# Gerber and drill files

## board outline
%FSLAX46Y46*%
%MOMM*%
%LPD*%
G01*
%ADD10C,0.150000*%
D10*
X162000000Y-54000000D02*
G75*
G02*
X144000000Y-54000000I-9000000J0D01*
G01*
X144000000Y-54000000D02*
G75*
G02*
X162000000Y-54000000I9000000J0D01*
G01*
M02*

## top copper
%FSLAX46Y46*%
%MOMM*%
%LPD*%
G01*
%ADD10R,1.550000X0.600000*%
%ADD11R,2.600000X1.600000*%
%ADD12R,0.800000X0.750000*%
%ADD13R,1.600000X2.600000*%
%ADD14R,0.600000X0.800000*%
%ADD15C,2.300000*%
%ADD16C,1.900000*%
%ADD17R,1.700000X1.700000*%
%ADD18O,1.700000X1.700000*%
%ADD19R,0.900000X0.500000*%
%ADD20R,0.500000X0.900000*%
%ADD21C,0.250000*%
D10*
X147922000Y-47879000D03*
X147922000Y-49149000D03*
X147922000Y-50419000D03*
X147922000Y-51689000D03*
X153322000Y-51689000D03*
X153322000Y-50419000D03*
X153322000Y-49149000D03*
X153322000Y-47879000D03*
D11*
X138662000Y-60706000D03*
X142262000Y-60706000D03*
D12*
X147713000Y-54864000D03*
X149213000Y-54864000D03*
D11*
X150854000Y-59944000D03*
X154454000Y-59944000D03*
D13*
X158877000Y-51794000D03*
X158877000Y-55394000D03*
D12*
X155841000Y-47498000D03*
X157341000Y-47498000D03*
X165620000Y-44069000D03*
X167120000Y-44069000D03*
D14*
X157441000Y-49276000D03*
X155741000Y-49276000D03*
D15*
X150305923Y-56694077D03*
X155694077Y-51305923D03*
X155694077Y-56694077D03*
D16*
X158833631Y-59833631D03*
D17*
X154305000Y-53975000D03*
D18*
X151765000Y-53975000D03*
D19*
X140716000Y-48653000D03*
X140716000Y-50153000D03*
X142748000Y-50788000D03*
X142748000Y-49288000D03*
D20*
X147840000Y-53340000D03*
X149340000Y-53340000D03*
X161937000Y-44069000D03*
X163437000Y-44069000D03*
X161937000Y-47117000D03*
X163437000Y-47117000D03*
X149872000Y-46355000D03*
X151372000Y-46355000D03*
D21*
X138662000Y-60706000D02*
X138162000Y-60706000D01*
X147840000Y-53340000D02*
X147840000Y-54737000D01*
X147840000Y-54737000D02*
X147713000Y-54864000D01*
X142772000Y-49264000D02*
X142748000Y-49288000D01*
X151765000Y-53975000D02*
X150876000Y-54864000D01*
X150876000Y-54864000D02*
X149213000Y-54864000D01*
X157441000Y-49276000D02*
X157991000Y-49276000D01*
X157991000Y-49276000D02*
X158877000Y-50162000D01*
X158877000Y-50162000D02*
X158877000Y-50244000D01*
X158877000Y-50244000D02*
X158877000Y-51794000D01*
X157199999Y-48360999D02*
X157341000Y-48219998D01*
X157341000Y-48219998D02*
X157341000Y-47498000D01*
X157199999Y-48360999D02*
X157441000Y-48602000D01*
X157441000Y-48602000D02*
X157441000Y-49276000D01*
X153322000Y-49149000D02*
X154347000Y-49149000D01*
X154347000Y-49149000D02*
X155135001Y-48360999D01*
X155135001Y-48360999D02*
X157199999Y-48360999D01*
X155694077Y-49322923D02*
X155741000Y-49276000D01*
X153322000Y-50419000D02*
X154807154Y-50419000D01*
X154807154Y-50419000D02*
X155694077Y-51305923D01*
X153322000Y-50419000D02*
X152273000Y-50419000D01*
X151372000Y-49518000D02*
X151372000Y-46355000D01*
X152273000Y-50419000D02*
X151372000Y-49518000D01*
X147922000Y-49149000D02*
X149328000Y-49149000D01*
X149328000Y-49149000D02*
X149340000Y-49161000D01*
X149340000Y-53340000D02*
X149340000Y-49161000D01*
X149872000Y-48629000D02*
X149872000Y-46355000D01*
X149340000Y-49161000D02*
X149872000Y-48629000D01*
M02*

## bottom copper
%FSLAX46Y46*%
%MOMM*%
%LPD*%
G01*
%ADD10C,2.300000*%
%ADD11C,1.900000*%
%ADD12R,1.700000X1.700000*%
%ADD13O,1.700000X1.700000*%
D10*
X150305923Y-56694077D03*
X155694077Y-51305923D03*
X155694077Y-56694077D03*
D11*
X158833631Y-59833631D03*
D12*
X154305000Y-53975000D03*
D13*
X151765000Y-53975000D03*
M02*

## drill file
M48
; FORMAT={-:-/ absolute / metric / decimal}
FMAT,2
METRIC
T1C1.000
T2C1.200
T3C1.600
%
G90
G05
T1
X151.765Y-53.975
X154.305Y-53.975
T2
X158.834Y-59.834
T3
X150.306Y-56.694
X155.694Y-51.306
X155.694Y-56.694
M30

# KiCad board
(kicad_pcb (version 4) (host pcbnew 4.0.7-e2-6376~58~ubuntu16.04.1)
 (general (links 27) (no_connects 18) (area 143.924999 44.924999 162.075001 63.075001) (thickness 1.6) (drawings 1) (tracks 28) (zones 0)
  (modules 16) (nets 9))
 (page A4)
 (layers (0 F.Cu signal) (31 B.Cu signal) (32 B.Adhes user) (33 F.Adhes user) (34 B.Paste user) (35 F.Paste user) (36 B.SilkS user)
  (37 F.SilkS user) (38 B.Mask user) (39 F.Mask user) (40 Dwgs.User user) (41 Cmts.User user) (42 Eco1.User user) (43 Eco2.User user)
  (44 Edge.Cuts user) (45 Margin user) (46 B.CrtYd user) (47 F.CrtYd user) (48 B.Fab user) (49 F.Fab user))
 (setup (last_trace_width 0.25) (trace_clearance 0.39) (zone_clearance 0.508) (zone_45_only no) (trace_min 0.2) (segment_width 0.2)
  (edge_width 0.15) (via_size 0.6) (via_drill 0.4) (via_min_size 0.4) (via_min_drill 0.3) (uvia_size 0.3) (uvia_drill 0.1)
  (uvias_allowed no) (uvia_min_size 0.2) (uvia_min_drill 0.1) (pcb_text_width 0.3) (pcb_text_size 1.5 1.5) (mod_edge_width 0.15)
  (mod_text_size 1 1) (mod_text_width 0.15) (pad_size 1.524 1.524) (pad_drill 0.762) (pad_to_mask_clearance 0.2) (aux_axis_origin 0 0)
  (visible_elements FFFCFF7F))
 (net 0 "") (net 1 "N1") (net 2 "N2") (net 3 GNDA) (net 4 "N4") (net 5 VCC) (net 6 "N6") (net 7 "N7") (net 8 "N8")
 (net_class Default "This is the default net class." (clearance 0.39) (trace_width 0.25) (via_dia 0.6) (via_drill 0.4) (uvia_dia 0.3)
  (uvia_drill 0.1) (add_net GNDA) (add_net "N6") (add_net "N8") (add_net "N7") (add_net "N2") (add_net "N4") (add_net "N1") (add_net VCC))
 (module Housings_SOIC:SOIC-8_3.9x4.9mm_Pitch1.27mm (layer F.Cu) (at 150.622 49.784)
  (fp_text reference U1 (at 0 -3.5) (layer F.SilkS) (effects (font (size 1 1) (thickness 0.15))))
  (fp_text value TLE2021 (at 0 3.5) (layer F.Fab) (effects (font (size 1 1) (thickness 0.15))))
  (pad 1 smd rect (at -2.7 -1.905) (size 1.55 0.6) (layers F.Cu F.Paste F.Mask))
  (pad 2 smd rect (at -2.7 -0.635) (size 1.55 0.6) (layers F.Cu F.Paste F.Mask) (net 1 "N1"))
  (pad 3 smd rect (at -2.7 0.635) (size 1.55 0.6) (layers F.Cu F.Paste F.Mask) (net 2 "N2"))
  (pad 4 smd rect (at -2.7 1.905) (size 1.55 0.6) (layers F.Cu F.Paste F.Mask) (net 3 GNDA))
  (pad 5 smd rect (at 2.7 1.905) (size 1.55 0.6) (layers F.Cu F.Paste F.Mask))
  (pad 6 smd rect (at 2.7 0.635) (size 1.55 0.6) (layers F.Cu F.Paste F.Mask) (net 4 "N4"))
  (pad 7 smd rect (at 2.7 -0.635) (size 1.55 0.6) (layers F.Cu F.Paste F.Mask) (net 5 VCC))
  (pad 8 smd rect (at 2.7 -1.905) (size 1.55 0.6) (layers F.Cu F.Paste F.Mask)))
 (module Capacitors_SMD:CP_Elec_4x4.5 (layer F.Cu) (at 140.462 60.706)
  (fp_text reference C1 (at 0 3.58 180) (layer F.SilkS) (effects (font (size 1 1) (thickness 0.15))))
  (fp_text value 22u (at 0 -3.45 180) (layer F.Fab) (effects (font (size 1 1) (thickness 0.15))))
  (pad 1 smd rect (at -1.8 0 180) (size 2.6 1.6) (layers F.Cu F.Paste F.Mask) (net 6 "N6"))
  (pad 2 smd rect (at 1.8 0 180) (size 2.6 1.6) (layers F.Cu F.Paste F.Mask) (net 3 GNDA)))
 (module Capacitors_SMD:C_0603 (layer F.Cu) (at 148.463 54.864 180)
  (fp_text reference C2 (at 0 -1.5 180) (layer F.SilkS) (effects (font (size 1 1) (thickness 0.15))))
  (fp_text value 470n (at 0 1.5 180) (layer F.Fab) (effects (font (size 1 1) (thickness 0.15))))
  (pad 2 smd rect (at 0.75 0 180) (size 0.8 0.75) (layers F.Cu F.Paste F.Mask) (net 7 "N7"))
  (pad 1 smd rect (at -0.75 0 180) (size 0.8 0.75) (layers F.Cu F.Paste F.Mask) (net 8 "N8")))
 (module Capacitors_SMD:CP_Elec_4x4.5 (layer F.Cu) (at 152.654 59.944)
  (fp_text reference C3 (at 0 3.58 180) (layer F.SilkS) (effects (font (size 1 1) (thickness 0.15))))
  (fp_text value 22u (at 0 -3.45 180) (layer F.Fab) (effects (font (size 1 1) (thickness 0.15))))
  (pad 1 smd rect (at -1.8 0 180) (size 2.6 1.6) (layers F.Cu F.Paste F.Mask) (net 2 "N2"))
  (pad 2 smd rect (at 1.8 0 180) (size 2.6 1.6) (layers F.Cu F.Paste F.Mask) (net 3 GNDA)))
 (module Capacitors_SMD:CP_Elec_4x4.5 (layer F.Cu) (at 158.877 53.594 270)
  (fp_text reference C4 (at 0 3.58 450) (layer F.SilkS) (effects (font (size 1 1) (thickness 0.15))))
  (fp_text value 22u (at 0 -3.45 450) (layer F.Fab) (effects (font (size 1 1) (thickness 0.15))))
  (pad 1 smd rect (at -1.8 0 90) (size 2.6 1.6) (layers F.Cu F.Paste F.Mask) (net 5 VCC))
  (pad 2 smd rect (at 1.8 0 90) (size 2.6 1.6) (layers F.Cu F.Paste F.Mask) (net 3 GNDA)))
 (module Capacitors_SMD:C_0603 (layer F.Cu) (at 156.591 47.498 180)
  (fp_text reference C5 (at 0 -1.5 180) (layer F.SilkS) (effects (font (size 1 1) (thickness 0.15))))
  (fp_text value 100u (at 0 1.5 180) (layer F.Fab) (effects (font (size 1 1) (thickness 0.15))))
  (pad 2 smd rect (at 0.75 0 180) (size 0.8 0.75) (layers F.Cu F.Paste F.Mask) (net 3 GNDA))
  (pad 1 smd rect (at -0.75 0 180) (size 0.8 0.75) (layers F.Cu F.Paste F.Mask) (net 5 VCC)))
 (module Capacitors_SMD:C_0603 (layer F.Cu) (at 166.37 44.069 180)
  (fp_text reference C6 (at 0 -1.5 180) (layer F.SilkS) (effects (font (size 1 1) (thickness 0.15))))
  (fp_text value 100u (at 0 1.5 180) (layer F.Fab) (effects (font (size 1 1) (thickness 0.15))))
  (pad 2 smd rect (at 0.75 0 180) (size 0.8 0.75) (layers F.Cu F.Paste F.Mask) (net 3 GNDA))
  (pad 1 smd rect (at -0.75 0 180) (size 0.8 0.75) (layers F.Cu F.Paste F.Mask) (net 5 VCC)))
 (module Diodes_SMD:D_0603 (layer F.Cu) (at 156.591 49.276 180)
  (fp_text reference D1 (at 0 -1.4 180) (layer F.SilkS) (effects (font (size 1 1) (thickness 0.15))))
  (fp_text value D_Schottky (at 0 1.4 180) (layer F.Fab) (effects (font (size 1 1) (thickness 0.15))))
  (pad 1 smd rect (at -0.85 0 180) (size 0.6 0.8) (layers F.Cu F.Paste F.Mask) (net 5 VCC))
  (pad 2 smd rect (at 0.85 0 180) (size 0.6 0.8) (layers F.Cu F.Paste F.Mask) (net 4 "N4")))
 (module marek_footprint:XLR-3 (layer B.Cu) (at 153 54 225)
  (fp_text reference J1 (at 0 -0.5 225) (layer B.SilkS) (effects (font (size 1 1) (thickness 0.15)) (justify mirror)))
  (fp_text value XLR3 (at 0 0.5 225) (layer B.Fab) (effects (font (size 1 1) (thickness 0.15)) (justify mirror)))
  (pad 1 thru_hole circle (at 3.81 0 225) (size 2.3 2.3) (drill 1.6) (layers *.Cu *.Mask) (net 3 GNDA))
  (pad 2 thru_hole circle (at -3.81 0 225) (size 2.3 2.3) (drill 1.6) (layers *.Cu *.Mask) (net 4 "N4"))
  (pad 3 thru_hole circle (at 0 -3.81 225) (size 2.3 2.3) (drill 1.6) (layers *.Cu *.Mask))
  (pad 4 thru_hole circle (at 0 -8.25 225) (size 1.9 1.9) (drill 1.2) (layers *.Cu *.Mask)))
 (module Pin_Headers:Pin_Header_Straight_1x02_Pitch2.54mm (layer F.Cu) (at 154.305 53.975 270)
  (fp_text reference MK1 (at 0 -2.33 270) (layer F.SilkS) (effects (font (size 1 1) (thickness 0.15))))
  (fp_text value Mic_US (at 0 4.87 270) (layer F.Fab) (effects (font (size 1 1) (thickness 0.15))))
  (pad 1 thru_hole rect (at 0 0 270) (size 1.7 1.7) (drill 1) (layers *.Cu *.Mask) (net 3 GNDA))
  (pad 2 thru_hole oval (at 0 2.54 270) (size 1.7 1.7) (drill 1) (layers *.Cu *.Mask) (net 8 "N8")))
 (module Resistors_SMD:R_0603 (layer F.Cu) (at 140.716 49.403 270)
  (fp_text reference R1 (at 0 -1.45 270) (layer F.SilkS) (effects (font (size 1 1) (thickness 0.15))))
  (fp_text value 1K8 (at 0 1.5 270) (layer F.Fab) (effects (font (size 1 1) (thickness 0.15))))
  (pad 1 smd rect (at -0.75 0 270) (size 0.5 0.9) (layers F.Cu F.Paste F.Mask) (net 5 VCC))
  (pad 2 smd rect (at 0.75 0 270) (size 0.5 0.9) (layers F.Cu F.Paste F.Mask) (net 6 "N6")))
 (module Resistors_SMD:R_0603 (layer F.Cu) (at 142.748 50.038 90)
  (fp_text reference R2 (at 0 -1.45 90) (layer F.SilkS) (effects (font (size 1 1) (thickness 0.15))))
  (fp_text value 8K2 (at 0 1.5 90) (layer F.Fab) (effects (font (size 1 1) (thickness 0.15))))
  (pad 1 smd rect (at -0.75 0 90) (size 0.5 0.9) (layers F.Cu F.Paste F.Mask) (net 6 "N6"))
  (pad 2 smd rect (at 0.75 0 90) (size 0.5 0.9) (layers F.Cu F.Paste F.Mask) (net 8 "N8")))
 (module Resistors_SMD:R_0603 (layer F.Cu) (at 148.59 53.34)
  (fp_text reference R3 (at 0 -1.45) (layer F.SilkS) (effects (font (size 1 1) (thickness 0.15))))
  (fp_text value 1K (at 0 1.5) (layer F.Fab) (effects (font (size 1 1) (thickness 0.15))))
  (pad 1 smd rect (at -0.75 0) (size 0.5 0.9) (layers F.Cu F.Paste F.Mask) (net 7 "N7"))
  (pad 2 smd rect (at 0.75 0) (size 0.5 0.9) (layers F.Cu F.Paste F.Mask) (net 1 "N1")))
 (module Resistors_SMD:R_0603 (layer F.Cu) (at 162.687 44.069)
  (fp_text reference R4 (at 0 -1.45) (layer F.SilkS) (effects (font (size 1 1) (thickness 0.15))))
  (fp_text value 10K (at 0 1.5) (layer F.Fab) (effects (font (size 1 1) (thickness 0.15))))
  (pad 1 smd rect (at -0.75 0) (size 0.5 0.9) (layers F.Cu F.Paste F.Mask) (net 5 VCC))
  (pad 2 smd rect (at 0.75 0) (size 0.5 0.9) (layers F.Cu F.Paste F.Mask) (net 2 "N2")))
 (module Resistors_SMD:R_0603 (layer F.Cu) (at 162.687 47.117)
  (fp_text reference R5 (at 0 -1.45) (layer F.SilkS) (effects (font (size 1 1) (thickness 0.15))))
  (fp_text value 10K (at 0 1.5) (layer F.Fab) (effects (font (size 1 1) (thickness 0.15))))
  (pad 1 smd rect (at -0.75 0) (size 0.5 0.9) (layers F.Cu F.Paste F.Mask) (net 2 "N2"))
  (pad 2 smd rect (at 0.75 0) (size 0.5 0.9) (layers F.Cu F.Paste F.Mask) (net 3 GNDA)))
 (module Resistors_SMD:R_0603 (layer F.Cu) (at 150.622 46.355)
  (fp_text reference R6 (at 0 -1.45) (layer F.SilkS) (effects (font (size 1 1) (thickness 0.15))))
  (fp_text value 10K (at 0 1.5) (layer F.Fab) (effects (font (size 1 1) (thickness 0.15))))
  (pad 1 smd rect (at -0.75 0) (size 0.5 0.9) (layers F.Cu F.Paste F.Mask) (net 1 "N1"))
  (pad 2 smd rect (at 0.75 0) (size 0.5 0.9) (layers F.Cu F.Paste F.Mask) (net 4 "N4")))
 (gr_circle (center 153 54) (end 162 54) (layer Edge.Cuts) (width 0.15))
 (segment (start 138.662 60.706) (end 138.162 60.706) (width 0.25) (layer F.Cu) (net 6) (status 30))
 (segment (start 147.84 53.34) (end 147.84 54.737) (width 0.25) (layer F.Cu) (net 7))
 (segment (start 147.84 54.737) (end 147.713 54.864) (width 0.25) (layer F.Cu) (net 7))
 (segment (start 142.772 49.264) (end 142.748 49.288) (width 0.25) (layer F.Cu) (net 8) (status 30))
 (segment (start 151.765 53.975) (end 150.876 54.864) (width 0.25) (layer F.Cu) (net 8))
 (segment (start 150.876 54.864) (end 149.213 54.864) (width 0.25) (layer F.Cu) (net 8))
 (segment (start 157.441 49.276) (end 157.991 49.276) (width 0.25) (layer F.Cu) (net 5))
 (segment (start 157.991 49.276) (end 158.877 50.162) (width 0.25) (layer F.Cu) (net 5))
 (segment (start 158.877 50.162) (end 158.877 50.244) (width 0.25) (layer F.Cu) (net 5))
 (segment (start 158.877 50.244) (end 158.877 51.794) (width 0.25) (layer F.Cu) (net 5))
 (segment (start 157.199999 48.360999) (end 157.341 48.219998) (width 0.25) (layer F.Cu) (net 5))
 (segment (start 157.341 48.219998) (end 157.341 47.498) (width 0.25) (layer F.Cu) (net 5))
 (segment (start 157.199999 48.360999) (end 157.441 48.602) (width 0.25) (layer F.Cu) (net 5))
 (segment (start 157.441 48.602) (end 157.441 49.276) (width 0.25) (layer F.Cu) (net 5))
 (segment (start 153.322 49.149) (end 154.347 49.149) (width 0.25) (layer F.Cu) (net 5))
 (segment (start 154.347 49.149) (end 155.135001 48.360999) (width 0.25) (layer F.Cu) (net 5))
 (segment (start 155.135001 48.360999) (end 157.199999 48.360999) (width 0.25) (layer F.Cu) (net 5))
 (segment (start 155.694077 49.322923) (end 155.741 49.276) (width 0.25) (layer F.Cu) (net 4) (status 30))
 (segment (start 153.322 50.419) (end 154.807154 50.419) (width 0.25) (layer F.Cu) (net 4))
 (segment (start 154.807154 50.419) (end 155.694077 51.305923) (width 0.25) (layer F.Cu) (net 4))
 (segment (start 153.322 50.419) (end 152.273 50.419) (width 0.25) (layer F.Cu) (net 4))
 (segment (start 151.372 49.518) (end 151.372 46.355) (width 0.25) (layer F.Cu) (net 4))
 (segment (start 152.273 50.419) (end 151.372 49.518) (width 0.25) (layer F.Cu) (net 4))
 (segment (start 147.922 49.149) (end 149.328 49.149) (width 0.25) (layer F.Cu) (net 1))
 (segment (start 149.328 49.149) (end 149.34 49.161) (width 0.25) (layer F.Cu) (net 1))
 (segment (start 149.34 53.34) (end 149.34 49.161) (width 0.25) (layer F.Cu) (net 1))
 (segment (start 149.872 48.629) (end 149.872 46.355) (width 0.25) (layer F.Cu) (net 1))
 (segment (start 149.34 49.161) (end 149.872 48.629) (width 0.25) (layer F.Cu) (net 1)))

